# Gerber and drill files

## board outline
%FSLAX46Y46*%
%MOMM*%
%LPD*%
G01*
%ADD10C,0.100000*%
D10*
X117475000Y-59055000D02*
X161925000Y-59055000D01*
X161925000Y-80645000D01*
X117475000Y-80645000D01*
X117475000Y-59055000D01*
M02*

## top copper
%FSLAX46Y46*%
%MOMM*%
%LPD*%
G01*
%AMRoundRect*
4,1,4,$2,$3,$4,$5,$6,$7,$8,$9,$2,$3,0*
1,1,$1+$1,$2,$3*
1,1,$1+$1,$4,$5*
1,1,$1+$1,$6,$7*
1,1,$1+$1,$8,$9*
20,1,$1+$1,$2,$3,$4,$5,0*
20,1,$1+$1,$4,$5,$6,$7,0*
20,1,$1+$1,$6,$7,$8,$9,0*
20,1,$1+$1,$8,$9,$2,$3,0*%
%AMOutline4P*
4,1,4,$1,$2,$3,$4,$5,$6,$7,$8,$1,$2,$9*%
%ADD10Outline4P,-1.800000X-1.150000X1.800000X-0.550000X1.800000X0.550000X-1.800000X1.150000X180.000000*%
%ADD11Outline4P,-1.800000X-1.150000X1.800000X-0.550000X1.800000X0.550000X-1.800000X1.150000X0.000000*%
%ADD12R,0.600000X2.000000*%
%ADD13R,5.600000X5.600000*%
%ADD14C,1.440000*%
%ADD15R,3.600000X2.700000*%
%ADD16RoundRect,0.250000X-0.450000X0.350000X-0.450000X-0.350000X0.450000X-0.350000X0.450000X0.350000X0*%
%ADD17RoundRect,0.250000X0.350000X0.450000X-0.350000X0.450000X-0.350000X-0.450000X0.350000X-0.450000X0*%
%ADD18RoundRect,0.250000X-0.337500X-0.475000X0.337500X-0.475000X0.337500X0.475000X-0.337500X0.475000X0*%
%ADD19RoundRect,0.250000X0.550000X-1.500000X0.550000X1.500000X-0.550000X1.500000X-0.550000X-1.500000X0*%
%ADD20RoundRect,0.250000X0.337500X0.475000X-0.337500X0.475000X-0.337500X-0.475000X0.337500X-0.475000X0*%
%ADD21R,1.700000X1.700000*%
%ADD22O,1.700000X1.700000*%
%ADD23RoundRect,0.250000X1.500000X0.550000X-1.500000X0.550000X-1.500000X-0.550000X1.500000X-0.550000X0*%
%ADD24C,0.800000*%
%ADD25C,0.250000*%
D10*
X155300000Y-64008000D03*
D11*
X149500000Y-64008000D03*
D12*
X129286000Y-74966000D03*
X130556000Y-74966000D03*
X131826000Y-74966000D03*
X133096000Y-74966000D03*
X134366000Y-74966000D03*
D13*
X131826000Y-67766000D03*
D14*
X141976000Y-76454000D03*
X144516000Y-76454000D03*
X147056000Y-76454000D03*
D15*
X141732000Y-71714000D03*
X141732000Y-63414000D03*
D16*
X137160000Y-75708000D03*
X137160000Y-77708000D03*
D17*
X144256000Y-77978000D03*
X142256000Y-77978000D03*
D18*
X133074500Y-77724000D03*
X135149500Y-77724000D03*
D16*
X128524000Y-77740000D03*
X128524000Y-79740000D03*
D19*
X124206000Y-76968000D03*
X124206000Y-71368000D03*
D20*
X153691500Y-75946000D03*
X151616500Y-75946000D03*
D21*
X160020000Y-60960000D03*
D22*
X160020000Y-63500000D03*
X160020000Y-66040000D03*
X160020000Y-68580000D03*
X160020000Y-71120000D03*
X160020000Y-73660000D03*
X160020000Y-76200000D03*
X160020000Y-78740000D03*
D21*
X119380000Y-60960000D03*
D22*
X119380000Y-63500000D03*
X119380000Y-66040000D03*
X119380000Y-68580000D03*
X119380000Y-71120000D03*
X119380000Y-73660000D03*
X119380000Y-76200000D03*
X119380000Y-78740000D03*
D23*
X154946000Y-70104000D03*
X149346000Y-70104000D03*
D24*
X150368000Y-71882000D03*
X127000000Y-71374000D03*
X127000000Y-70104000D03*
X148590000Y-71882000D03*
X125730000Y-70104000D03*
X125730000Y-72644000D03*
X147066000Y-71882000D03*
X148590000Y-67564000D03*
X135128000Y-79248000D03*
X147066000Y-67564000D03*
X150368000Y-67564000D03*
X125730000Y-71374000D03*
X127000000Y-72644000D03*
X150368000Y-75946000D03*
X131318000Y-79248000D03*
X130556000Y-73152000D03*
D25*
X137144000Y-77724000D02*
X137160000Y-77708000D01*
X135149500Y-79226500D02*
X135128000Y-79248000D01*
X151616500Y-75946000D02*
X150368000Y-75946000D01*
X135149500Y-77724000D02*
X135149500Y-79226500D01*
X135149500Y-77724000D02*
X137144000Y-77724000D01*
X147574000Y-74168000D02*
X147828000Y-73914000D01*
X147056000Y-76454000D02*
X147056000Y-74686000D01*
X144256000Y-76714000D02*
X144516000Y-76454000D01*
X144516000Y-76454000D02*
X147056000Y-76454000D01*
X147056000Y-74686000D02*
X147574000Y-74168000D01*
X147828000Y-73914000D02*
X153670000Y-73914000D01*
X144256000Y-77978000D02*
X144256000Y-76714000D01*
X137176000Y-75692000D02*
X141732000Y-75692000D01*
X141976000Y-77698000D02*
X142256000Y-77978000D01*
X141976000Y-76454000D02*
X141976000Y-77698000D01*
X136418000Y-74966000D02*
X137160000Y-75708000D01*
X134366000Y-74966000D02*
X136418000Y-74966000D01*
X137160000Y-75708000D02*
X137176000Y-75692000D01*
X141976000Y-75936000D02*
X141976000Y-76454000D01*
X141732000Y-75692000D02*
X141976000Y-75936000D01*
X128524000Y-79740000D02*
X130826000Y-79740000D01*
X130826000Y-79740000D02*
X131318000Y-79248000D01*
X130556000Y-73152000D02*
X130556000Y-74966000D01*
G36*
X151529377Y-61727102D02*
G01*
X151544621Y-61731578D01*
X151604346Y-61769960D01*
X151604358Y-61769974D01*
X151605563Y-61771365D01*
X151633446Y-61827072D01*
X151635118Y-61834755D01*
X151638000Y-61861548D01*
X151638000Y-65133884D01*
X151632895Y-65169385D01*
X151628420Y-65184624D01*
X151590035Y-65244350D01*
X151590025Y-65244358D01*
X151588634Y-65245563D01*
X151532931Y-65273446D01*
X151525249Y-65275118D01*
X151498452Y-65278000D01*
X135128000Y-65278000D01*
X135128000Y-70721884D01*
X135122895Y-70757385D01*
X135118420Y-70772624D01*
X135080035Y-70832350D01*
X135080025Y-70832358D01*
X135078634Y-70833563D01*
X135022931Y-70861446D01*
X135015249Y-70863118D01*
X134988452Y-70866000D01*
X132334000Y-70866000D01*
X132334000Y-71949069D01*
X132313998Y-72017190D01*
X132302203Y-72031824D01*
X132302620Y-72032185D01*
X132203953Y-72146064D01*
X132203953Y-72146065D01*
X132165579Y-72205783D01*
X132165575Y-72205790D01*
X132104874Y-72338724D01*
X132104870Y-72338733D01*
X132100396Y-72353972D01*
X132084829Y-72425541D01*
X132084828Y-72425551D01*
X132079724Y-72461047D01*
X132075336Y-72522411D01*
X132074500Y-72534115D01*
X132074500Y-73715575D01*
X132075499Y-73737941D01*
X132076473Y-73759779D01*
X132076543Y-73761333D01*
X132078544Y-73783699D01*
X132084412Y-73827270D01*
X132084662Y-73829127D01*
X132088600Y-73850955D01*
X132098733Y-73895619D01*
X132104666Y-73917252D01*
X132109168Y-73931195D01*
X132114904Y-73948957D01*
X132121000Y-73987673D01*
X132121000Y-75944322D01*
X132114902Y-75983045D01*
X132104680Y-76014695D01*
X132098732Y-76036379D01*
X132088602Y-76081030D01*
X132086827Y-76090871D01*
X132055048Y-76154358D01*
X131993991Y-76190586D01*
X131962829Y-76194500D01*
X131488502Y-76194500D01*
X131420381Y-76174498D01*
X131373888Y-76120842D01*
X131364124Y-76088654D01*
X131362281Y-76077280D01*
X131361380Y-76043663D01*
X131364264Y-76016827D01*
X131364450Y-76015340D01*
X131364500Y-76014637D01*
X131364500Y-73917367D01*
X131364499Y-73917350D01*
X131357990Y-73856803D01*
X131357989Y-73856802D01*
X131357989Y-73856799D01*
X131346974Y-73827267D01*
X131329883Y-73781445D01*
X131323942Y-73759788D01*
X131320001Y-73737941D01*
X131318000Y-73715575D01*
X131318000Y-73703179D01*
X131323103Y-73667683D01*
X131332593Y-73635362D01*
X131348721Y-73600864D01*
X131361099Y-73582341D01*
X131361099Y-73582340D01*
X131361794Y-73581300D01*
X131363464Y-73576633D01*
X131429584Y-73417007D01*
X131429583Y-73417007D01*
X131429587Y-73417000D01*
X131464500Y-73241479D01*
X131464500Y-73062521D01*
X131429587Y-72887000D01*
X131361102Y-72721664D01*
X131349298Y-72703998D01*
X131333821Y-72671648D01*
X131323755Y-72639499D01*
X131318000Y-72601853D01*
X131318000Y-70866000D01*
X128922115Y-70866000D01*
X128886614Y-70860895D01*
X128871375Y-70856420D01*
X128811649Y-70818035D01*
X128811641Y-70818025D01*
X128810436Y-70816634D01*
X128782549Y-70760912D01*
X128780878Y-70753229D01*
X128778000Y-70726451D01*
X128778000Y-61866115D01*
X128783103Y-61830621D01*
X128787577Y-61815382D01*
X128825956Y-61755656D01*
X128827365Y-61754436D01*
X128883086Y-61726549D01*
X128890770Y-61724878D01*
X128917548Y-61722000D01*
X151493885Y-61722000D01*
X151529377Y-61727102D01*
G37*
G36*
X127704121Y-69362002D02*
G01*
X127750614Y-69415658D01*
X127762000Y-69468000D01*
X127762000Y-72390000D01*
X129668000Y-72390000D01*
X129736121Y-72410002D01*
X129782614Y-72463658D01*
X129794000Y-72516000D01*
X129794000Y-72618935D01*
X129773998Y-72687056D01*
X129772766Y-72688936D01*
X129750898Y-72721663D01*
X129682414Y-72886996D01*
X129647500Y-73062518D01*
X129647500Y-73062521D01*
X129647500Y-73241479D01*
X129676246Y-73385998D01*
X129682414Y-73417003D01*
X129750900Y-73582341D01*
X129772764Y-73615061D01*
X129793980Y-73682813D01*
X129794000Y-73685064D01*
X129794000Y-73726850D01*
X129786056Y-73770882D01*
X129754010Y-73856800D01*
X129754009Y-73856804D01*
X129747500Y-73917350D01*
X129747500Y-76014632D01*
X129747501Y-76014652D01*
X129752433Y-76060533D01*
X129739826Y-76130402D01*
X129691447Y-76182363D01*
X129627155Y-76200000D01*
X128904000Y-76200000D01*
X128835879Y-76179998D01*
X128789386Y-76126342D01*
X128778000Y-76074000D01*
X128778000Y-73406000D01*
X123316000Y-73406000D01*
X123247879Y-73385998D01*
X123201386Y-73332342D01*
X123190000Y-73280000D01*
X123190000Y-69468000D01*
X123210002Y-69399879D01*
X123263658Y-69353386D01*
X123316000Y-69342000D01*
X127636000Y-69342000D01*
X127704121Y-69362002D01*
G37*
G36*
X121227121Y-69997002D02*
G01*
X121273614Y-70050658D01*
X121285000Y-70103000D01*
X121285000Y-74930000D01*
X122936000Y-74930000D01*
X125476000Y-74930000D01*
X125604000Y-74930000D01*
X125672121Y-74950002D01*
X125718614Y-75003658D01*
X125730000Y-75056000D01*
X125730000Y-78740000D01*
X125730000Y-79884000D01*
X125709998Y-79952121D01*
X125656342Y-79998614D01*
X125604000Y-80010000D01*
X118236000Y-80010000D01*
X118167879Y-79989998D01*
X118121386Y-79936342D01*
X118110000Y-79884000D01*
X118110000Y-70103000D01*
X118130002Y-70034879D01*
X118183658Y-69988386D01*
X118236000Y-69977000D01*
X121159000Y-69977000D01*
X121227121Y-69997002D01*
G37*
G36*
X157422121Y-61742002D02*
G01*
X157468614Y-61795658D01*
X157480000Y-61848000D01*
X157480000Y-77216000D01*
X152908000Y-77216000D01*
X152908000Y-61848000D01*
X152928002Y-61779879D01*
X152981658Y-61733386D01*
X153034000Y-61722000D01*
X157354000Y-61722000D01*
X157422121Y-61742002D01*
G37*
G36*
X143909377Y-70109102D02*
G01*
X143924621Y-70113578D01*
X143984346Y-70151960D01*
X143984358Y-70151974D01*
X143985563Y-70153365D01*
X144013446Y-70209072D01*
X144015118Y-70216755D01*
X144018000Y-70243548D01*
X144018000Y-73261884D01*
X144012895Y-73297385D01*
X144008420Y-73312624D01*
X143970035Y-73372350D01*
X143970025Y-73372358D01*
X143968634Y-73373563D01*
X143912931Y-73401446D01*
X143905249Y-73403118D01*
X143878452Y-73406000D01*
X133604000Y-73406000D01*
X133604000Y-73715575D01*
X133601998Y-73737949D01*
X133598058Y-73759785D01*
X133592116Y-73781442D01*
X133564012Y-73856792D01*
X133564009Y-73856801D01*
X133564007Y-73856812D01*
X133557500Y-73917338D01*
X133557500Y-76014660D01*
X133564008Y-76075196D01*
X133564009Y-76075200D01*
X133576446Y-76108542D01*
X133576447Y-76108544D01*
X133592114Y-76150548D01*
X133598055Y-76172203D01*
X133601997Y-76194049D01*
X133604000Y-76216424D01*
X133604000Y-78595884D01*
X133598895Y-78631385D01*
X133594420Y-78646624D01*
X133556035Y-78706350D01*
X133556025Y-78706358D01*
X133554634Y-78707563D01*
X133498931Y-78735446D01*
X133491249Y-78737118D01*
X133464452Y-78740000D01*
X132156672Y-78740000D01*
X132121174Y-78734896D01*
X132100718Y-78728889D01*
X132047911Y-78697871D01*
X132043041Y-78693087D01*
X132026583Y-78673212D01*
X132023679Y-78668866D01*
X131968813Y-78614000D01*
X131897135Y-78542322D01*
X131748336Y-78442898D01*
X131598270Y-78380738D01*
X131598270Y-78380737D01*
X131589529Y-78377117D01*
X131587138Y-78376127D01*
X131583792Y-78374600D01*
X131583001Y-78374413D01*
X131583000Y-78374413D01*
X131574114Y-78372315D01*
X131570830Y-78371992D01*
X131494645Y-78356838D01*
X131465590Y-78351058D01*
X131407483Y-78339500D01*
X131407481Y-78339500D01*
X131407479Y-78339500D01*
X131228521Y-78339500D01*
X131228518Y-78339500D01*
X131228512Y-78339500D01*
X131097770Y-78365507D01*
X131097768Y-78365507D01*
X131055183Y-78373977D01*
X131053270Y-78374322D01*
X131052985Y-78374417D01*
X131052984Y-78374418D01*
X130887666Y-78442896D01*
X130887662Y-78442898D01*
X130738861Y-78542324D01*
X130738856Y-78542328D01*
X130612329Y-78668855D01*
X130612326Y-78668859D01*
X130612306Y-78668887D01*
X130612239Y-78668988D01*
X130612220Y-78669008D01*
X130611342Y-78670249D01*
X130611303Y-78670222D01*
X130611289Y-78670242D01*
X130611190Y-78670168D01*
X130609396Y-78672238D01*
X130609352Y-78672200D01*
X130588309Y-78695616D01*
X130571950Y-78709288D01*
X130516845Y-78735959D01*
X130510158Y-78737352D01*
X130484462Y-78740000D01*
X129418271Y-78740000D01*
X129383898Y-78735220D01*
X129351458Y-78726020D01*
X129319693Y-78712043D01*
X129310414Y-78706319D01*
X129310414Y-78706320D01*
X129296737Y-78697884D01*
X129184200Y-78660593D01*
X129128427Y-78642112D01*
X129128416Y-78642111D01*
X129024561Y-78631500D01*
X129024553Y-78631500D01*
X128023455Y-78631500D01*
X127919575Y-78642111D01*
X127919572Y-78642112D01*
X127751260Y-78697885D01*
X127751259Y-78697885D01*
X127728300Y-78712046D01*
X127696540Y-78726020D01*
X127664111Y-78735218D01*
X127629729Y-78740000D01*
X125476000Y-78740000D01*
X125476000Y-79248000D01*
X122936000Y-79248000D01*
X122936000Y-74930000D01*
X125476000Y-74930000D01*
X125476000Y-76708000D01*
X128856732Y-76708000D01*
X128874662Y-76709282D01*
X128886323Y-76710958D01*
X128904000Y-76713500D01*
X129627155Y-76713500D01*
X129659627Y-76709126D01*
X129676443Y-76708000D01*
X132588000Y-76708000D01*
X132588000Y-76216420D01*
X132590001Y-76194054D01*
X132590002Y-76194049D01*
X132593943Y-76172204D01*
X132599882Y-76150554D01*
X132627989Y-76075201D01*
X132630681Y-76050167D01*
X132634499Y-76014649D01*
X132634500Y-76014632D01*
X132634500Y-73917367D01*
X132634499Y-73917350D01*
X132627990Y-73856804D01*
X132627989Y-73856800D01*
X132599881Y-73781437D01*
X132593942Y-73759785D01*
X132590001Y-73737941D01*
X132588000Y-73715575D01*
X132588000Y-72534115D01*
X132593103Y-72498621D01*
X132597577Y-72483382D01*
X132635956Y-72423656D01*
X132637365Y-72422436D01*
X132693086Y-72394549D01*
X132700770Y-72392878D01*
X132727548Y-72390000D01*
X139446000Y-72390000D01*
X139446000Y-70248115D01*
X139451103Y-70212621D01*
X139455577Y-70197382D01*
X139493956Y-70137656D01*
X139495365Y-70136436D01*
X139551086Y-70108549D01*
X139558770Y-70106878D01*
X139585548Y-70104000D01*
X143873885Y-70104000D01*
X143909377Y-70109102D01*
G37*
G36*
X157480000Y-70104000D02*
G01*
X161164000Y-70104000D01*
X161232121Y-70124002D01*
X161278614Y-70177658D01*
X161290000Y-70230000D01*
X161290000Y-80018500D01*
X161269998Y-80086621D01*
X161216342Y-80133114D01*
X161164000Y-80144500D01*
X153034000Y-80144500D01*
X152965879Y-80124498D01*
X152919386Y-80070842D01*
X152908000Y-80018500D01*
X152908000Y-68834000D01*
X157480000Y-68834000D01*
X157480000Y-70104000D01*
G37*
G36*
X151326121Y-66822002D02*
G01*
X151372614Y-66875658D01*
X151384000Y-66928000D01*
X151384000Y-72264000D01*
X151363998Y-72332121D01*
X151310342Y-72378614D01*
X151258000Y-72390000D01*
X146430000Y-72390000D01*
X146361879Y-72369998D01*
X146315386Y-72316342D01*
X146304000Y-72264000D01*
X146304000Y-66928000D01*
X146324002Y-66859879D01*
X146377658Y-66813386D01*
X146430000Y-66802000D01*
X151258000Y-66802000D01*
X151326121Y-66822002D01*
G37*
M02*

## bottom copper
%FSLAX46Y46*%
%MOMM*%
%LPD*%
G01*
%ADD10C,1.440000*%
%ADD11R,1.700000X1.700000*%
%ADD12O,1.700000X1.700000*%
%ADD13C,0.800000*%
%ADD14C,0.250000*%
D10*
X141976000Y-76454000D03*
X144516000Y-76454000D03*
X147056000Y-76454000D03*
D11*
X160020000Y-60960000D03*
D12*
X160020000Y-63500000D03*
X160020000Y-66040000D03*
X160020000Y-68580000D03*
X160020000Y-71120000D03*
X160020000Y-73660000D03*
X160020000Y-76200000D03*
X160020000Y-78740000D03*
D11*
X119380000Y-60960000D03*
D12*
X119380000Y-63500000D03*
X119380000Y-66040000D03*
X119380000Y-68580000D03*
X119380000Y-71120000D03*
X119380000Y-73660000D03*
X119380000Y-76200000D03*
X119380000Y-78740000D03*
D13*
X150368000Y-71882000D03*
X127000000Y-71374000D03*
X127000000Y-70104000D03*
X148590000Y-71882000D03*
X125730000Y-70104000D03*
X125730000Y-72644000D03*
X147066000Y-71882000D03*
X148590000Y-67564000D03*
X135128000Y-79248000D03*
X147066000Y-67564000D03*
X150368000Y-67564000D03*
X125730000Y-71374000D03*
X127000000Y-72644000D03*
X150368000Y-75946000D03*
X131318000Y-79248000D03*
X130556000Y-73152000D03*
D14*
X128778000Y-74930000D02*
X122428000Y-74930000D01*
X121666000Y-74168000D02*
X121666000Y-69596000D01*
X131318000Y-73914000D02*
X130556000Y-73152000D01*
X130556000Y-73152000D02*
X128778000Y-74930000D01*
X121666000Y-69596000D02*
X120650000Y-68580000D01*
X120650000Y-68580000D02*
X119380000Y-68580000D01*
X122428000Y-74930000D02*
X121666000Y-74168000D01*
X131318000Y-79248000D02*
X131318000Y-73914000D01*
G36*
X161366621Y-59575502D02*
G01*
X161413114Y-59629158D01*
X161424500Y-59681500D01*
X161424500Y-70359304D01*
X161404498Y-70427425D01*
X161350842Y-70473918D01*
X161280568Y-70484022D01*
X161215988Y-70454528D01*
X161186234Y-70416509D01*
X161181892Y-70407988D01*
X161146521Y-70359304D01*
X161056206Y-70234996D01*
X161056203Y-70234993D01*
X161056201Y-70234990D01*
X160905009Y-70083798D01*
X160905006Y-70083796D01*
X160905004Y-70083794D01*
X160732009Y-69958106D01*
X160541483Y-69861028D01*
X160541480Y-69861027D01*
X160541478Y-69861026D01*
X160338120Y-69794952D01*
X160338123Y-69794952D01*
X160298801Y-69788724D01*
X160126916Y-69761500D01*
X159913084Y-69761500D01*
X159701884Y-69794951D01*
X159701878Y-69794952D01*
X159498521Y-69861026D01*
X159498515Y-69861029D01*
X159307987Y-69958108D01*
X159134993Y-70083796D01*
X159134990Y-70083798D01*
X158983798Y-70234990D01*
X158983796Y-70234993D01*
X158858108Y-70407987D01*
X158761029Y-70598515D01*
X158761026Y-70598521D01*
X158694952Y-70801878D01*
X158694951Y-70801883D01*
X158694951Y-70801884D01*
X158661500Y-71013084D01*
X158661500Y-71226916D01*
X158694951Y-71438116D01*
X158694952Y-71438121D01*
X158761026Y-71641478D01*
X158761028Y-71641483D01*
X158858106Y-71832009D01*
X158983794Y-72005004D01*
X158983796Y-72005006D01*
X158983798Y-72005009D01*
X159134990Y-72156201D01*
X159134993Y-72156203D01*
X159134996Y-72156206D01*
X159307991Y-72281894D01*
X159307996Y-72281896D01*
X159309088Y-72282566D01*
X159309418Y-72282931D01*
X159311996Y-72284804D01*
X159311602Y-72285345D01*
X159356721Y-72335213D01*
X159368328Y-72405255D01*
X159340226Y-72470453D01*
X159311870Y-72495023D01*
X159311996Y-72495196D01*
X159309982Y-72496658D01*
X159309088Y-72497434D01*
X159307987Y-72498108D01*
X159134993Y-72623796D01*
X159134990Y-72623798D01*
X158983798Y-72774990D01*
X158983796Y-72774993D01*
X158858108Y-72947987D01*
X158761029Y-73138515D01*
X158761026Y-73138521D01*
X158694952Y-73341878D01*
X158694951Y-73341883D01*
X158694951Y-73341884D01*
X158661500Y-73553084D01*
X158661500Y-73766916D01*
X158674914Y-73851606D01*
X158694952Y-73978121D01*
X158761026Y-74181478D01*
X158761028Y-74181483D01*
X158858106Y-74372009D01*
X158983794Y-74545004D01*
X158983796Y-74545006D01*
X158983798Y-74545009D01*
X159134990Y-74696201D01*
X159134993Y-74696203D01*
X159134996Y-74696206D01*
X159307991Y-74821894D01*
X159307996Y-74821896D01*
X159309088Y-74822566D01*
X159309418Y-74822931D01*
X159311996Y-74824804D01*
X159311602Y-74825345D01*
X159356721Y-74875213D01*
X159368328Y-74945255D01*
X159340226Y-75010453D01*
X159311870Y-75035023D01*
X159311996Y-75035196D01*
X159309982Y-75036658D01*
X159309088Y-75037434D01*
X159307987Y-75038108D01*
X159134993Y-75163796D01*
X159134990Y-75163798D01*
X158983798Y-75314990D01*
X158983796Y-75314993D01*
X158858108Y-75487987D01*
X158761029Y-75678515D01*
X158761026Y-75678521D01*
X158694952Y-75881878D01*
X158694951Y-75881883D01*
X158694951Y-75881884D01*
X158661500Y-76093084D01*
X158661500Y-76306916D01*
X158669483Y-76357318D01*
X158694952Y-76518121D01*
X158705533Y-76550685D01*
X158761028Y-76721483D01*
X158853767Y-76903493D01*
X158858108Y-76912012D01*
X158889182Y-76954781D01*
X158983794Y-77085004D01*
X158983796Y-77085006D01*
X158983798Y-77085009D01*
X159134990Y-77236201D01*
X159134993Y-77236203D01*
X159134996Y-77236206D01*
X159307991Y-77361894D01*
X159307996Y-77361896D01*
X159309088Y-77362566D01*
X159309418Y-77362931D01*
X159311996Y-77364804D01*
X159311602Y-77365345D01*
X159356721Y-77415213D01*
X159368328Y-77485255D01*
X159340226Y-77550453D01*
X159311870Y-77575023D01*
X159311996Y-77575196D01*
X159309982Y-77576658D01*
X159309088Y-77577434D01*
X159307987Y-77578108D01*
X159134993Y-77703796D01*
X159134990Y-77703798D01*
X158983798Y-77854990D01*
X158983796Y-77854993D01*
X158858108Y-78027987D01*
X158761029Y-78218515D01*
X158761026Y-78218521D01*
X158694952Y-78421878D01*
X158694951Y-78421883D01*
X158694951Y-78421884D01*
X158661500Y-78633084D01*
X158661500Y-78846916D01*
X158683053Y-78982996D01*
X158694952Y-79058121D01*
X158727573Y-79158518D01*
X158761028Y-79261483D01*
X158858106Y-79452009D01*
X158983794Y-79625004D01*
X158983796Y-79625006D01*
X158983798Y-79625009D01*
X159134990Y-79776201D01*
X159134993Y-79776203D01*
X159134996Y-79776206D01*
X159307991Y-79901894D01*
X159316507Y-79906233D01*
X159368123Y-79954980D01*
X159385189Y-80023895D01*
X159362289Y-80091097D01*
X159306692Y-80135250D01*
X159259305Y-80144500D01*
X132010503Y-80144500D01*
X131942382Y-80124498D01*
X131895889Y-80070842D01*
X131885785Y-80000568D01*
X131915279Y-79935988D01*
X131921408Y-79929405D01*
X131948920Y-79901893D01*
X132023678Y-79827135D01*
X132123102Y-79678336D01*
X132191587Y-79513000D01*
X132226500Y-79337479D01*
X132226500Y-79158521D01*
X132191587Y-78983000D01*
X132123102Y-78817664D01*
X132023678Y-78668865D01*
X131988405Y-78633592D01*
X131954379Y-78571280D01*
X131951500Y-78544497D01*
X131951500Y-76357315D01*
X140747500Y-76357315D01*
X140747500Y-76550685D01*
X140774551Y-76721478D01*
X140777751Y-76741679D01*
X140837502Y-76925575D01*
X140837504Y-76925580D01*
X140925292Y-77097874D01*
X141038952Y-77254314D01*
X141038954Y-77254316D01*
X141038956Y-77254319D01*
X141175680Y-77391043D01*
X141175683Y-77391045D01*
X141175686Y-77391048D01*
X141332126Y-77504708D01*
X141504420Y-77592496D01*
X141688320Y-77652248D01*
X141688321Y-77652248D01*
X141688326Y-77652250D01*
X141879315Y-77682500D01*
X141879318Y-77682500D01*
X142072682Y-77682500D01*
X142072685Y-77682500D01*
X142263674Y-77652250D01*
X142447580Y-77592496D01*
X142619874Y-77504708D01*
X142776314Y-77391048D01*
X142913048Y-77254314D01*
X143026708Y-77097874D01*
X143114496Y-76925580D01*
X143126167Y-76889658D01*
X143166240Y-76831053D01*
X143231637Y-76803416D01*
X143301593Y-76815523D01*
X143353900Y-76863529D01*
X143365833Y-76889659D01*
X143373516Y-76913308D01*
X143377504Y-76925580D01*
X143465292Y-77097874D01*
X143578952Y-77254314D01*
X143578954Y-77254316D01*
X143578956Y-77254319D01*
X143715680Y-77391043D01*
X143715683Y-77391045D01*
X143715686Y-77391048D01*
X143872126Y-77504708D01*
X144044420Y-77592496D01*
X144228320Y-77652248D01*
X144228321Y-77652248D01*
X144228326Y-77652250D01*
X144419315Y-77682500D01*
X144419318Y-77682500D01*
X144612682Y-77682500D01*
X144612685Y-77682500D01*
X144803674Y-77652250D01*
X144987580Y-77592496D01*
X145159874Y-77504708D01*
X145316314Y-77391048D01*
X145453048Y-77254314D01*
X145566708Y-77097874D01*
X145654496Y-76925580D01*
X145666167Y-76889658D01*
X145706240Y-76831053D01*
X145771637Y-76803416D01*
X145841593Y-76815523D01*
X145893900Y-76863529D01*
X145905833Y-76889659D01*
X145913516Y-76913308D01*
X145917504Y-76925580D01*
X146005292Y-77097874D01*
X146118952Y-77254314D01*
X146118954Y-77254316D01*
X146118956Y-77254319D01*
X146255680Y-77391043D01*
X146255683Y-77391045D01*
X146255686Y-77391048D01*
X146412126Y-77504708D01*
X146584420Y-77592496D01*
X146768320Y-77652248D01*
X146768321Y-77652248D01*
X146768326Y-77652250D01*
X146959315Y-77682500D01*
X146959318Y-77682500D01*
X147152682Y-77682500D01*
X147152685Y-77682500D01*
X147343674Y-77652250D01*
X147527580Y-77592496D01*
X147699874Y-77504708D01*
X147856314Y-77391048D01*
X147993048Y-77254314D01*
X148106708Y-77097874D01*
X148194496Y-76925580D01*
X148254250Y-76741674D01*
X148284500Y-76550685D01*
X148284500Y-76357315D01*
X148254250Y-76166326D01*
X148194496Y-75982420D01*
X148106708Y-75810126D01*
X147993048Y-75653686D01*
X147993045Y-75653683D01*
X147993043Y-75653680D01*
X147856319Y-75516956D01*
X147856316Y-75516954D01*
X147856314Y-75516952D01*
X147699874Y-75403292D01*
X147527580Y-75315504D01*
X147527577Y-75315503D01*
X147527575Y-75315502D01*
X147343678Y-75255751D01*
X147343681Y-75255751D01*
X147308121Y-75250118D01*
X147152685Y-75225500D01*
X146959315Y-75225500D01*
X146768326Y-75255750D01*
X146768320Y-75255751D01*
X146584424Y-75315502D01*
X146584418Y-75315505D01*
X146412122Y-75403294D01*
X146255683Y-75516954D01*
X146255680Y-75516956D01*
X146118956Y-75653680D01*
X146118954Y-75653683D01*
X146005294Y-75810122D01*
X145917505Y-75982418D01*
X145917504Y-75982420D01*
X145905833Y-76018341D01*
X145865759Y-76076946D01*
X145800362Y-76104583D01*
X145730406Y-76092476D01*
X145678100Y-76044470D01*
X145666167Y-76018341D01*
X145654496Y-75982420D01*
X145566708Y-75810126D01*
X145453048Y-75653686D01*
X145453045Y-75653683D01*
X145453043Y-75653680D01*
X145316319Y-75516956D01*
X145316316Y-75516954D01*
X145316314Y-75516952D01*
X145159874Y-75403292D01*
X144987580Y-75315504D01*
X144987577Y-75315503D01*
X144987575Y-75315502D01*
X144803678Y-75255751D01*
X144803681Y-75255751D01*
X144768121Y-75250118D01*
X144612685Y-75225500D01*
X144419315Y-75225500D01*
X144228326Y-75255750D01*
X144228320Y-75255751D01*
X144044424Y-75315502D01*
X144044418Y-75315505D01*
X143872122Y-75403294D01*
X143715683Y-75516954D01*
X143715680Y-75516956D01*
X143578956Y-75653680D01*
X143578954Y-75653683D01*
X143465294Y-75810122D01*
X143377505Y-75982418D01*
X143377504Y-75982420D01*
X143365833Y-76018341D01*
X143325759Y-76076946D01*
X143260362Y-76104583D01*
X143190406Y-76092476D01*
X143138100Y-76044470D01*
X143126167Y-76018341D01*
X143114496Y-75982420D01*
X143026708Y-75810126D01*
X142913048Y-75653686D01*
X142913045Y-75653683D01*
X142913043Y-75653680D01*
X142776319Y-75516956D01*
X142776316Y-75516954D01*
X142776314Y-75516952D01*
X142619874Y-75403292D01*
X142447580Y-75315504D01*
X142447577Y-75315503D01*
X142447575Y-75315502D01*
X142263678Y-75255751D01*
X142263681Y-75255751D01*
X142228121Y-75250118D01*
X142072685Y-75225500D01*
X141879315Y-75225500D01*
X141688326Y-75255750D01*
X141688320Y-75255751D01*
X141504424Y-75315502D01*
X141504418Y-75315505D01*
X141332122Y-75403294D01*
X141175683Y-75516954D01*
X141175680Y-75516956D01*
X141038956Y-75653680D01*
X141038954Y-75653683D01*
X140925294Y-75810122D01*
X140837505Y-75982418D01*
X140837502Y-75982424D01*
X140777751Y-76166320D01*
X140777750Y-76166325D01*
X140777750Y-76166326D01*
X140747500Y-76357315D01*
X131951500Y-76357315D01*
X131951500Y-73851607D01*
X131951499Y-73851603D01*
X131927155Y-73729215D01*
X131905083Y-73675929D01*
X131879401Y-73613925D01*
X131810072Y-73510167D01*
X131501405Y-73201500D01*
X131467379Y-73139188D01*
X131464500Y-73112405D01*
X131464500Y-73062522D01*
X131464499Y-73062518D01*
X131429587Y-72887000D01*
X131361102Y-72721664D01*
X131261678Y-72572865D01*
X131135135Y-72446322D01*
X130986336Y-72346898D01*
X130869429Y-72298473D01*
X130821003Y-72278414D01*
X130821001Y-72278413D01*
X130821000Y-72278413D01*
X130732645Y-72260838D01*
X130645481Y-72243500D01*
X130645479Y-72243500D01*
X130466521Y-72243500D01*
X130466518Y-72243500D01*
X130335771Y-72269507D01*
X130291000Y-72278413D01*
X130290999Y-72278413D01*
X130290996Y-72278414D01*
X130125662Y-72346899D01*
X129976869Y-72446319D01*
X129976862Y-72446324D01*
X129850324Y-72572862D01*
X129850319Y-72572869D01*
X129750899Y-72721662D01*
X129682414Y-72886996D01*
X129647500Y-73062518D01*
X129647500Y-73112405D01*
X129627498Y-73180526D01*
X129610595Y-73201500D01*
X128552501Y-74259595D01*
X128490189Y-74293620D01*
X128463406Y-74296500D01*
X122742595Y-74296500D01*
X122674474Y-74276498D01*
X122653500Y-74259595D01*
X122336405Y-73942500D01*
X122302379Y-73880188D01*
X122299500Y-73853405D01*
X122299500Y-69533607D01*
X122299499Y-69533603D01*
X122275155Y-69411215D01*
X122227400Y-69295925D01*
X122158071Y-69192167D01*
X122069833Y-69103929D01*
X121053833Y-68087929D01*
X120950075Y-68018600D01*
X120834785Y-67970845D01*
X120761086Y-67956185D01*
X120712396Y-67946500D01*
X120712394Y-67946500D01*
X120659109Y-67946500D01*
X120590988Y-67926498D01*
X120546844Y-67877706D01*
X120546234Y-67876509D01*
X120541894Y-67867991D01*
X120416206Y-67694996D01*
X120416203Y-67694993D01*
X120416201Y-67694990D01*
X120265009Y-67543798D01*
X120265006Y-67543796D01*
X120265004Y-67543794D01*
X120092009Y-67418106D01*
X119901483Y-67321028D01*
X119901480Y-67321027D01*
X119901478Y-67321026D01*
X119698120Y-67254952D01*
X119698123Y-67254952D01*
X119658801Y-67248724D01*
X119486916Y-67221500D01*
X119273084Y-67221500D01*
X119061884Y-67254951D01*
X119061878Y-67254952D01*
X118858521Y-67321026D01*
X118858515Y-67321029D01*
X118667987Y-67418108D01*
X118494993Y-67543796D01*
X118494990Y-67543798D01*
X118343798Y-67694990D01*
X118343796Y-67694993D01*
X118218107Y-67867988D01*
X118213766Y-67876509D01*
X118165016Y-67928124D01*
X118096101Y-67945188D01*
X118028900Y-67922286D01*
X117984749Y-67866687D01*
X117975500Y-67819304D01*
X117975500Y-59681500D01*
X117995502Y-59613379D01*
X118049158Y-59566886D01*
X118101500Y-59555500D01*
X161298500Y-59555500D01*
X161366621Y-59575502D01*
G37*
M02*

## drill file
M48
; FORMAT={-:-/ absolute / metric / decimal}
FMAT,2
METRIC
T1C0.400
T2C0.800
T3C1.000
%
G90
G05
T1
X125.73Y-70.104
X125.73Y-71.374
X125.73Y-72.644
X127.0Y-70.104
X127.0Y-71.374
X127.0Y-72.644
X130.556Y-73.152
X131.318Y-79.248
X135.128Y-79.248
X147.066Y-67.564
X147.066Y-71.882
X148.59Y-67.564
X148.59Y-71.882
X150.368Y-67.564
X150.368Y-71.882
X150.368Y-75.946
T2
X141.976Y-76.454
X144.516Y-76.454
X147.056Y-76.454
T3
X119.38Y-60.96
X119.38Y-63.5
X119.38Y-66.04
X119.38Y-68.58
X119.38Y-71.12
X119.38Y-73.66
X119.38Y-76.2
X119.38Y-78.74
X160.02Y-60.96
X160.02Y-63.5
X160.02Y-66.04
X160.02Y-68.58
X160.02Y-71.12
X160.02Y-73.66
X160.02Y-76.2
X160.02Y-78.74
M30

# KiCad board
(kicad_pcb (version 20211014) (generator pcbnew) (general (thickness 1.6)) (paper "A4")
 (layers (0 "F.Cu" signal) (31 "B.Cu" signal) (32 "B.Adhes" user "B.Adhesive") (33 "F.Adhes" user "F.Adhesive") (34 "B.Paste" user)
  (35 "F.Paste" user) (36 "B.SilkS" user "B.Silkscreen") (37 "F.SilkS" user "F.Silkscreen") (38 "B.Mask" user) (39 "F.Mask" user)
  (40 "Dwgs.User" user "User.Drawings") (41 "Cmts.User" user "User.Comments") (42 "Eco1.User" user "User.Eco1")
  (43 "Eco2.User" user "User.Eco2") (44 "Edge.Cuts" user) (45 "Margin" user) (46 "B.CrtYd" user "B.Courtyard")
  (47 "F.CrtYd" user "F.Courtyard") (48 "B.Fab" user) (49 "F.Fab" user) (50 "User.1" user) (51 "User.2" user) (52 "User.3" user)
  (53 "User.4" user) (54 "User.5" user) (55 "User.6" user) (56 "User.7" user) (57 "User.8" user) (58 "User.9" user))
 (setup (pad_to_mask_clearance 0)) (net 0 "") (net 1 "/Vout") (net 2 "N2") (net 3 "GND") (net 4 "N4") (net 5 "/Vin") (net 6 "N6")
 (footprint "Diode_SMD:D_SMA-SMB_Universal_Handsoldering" (layer "F.Cu") (at 152.4 64.008 180)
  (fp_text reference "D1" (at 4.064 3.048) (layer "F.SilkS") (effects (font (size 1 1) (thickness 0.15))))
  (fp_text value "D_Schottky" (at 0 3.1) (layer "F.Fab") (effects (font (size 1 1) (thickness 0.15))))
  (pad "1" smd trapezoid locked (at -2.9 0 180) (size 3.6 1.7) (rect_delta 0.6 0) (layers "F.Cu" "F.Paste" "F.Mask") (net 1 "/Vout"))
  (pad "2" smd trapezoid locked (at 2.9 0) (size 3.6 1.7) (rect_delta 0.6 0) (layers "F.Cu" "F.Paste" "F.Mask") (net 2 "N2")))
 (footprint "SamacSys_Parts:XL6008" (layer "F.Cu") (at 131.826 74.966)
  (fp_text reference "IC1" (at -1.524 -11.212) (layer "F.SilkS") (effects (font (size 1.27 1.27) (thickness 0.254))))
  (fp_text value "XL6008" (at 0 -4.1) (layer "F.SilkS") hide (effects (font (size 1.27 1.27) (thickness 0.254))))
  (pad "1" smd rect locked (at -2.54 0) (size 0.6 2) (layers "F.Cu" "F.Paste" "F.Mask") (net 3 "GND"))
  (pad "2" smd rect locked (at -1.27 0) (size 0.6 2) (layers "F.Cu" "F.Paste" "F.Mask") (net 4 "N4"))
  (pad "3" smd rect locked (at 0 0) (size 0.6 2) (layers "F.Cu" "F.Paste" "F.Mask") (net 2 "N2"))
  (pad "4" smd rect locked (at 1.27 0) (size 0.6 2) (layers "F.Cu" "F.Paste" "F.Mask") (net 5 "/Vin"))
  (pad "5" smd rect locked (at 2.54 0) (size 0.6 2) (layers "F.Cu" "F.Paste" "F.Mask") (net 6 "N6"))
  (pad "6" smd rect locked (at 0 -7.2 90) (size 5.6 5.6) (layers "F.Cu" "F.Paste" "F.Mask") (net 2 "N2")))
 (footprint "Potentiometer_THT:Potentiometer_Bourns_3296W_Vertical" (layer "F.Cu") (at 141.976 76.454 180)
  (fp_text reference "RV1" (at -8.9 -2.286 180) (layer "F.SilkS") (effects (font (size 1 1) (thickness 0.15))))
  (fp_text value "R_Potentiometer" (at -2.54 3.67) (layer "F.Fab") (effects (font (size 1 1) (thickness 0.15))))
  (pad "1" thru_hole circle locked (at 0 0 180) (size 1.44 1.44) (drill 0.8) (layers *.Cu *.Mask) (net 6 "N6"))
  (pad "2" thru_hole circle locked (at -2.54 0 180) (size 1.44 1.44) (drill 0.8) (layers *.Cu *.Mask) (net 1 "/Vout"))
  (pad "3" thru_hole circle locked (at -5.08 0 180) (size 1.44 1.44) (drill 0.8) (layers *.Cu *.Mask) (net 1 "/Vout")))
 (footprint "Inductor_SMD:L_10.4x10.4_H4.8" (layer "F.Cu") (at 141.732 67.564 90)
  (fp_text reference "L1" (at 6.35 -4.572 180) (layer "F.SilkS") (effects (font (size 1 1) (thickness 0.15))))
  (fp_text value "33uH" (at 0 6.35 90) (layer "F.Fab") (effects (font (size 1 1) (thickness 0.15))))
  (pad "1" smd rect locked (at -4.15 0 90) (size 2.7 3.6) (layers "F.Cu" "F.Paste" "F.Mask") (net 5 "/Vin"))
  (pad "2" smd rect locked (at 4.15 0 90) (size 2.7 3.6) (layers "F.Cu" "F.Paste" "F.Mask") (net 2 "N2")))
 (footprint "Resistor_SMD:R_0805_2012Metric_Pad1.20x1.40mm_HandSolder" (layer "F.Cu") (at 137.16 76.708 -90)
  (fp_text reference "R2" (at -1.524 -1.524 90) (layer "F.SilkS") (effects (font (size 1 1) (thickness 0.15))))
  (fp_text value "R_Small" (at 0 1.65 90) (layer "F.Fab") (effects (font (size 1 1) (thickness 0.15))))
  (pad "1" smd roundrect locked (at -1 0 270) (size 1.2 1.4) (layers "F.Cu" "F.Paste" "F.Mask") (roundrect_rratio 0.208333) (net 6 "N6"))
  (pad "2" smd roundrect locked (at 1 0 270) (size 1.2 1.4) (layers "F.Cu" "F.Paste" "F.Mask") (roundrect_rratio 0.208333) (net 3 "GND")))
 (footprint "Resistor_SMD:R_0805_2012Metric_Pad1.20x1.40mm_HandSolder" (layer "F.Cu") (at 143.256 77.978 180)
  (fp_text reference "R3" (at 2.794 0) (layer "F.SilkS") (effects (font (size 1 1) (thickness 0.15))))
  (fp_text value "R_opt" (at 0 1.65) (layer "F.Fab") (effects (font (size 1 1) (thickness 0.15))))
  (pad "1" smd roundrect locked (at -1 0 180) (size 1.2 1.4) (layers "F.Cu" "F.Paste" "F.Mask") (roundrect_rratio 0.208333) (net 1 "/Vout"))
  (pad "2" smd roundrect locked (at 1 0 180) (size 1.2 1.4) (layers "F.Cu" "F.Paste" "F.Mask") (roundrect_rratio 0.208333) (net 6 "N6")))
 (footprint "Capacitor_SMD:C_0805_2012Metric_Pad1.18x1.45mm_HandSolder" (layer "F.Cu") (at 134.112 77.724)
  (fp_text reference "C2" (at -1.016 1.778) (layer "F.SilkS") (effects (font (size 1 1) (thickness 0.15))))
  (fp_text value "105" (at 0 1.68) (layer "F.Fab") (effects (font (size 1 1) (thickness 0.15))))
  (pad "1" smd roundrect locked (at -1.0375 0) (size 1.175 1.45) (layers "F.Cu" "F.Paste" "F.Mask") (roundrect_rratio 0.212766)
   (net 5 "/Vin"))
  (pad "2" smd roundrect locked (at 1.0375 0) (size 1.175 1.45) (layers "F.Cu" "F.Paste" "F.Mask") (roundrect_rratio 0.212766) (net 3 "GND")))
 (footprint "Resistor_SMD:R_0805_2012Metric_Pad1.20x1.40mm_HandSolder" (layer "F.Cu") (at 128.524 78.74 -90)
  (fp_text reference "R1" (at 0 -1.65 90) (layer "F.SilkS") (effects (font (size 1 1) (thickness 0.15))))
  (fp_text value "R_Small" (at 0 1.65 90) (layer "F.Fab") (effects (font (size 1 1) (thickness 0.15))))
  (pad "1" smd roundrect locked (at -1 0 270) (size 1.2 1.4) (layers "F.Cu" "F.Paste" "F.Mask") (roundrect_rratio 0.208333) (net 5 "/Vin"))
  (pad "2" smd roundrect locked (at 1 0 270) (size 1.2 1.4) (layers "F.Cu" "F.Paste" "F.Mask") (roundrect_rratio 0.208333) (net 4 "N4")))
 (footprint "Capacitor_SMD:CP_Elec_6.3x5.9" (layer "F.Cu") (at 124.206 74.168 90)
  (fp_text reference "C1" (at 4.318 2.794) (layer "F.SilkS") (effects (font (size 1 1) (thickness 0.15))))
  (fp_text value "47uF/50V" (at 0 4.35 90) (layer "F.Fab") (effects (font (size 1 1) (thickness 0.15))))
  (pad "1" smd roundrect locked (at -2.8 0 90) (size 3.5 1.6) (layers "F.Cu" "F.Paste" "F.Mask") (roundrect_rratio 0.15625) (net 5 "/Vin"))
  (pad "2" smd roundrect locked (at 2.8 0 90) (size 3.5 1.6) (layers "F.Cu" "F.Paste" "F.Mask") (roundrect_rratio 0.15625) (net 3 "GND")))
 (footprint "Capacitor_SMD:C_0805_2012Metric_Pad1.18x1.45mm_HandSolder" (layer "F.Cu") (at 152.654 75.946 180)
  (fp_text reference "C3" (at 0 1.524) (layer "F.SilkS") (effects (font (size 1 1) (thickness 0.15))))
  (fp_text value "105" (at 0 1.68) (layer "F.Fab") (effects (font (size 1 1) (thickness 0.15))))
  (pad "1" smd roundrect locked (at -1.0375 0 180) (size 1.175 1.45) (layers "F.Cu" "F.Paste" "F.Mask") (roundrect_rratio 0.212766)
   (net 1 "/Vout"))
  (pad "2" smd roundrect locked (at 1.0375 0 180) (size 1.175 1.45) (layers "F.Cu" "F.Paste" "F.Mask") (roundrect_rratio 0.212766)
   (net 3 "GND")))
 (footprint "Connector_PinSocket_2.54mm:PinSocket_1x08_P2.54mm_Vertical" (layer "F.Cu") (at 160.02 60.96)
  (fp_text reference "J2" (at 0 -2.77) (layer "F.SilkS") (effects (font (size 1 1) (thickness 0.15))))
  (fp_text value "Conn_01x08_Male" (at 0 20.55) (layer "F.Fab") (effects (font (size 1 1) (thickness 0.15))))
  (pad "1" thru_hole rect locked (at 0 0) (size 1.7 1.7) (drill 1) (layers *.Cu *.Mask) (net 3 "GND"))
  (pad "2" thru_hole oval locked (at 0 2.54) (size 1.7 1.7) (drill 1) (layers *.Cu *.Mask) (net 3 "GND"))
  (pad "3" thru_hole oval locked (at 0 5.08) (size 1.7 1.7) (drill 1) (layers *.Cu *.Mask) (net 3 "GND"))
  (pad "4" thru_hole oval locked (at 0 7.62) (size 1.7 1.7) (drill 1) (layers *.Cu *.Mask) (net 3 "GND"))
  (pad "5" thru_hole oval locked (at 0 10.16) (size 1.7 1.7) (drill 1) (layers *.Cu *.Mask) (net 1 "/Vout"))
  (pad "6" thru_hole oval locked (at 0 12.7) (size 1.7 1.7) (drill 1) (layers *.Cu *.Mask) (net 1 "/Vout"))
  (pad "7" thru_hole oval locked (at 0 15.24) (size 1.7 1.7) (drill 1) (layers *.Cu *.Mask) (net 1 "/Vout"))
  (pad "8" thru_hole oval locked (at 0 17.78) (size 1.7 1.7) (drill 1) (layers *.Cu *.Mask) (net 1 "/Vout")))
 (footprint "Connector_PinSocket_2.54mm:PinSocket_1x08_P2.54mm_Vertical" (layer "F.Cu") (at 119.38 60.96)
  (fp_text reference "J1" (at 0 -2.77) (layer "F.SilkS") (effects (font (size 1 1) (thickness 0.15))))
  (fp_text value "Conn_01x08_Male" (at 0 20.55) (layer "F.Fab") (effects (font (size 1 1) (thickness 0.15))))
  (pad "1" thru_hole rect locked (at 0 0) (size 1.7 1.7) (drill 1) (layers *.Cu *.Mask) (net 3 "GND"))
  (pad "2" thru_hole oval locked (at 0 2.54) (size 1.7 1.7) (drill 1) (layers *.Cu *.Mask) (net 3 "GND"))
  (pad "3" thru_hole oval locked (at 0 5.08) (size 1.7 1.7) (drill 1) (layers *.Cu *.Mask) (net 3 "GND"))
  (pad "4" thru_hole oval locked (at 0 7.62) (size 1.7 1.7) (drill 1) (layers *.Cu *.Mask) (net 4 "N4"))
  (pad "5" thru_hole oval locked (at 0 10.16) (size 1.7 1.7) (drill 1) (layers *.Cu *.Mask) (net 5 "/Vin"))
  (pad "6" thru_hole oval locked (at 0 12.7) (size 1.7 1.7) (drill 1) (layers *.Cu *.Mask) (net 5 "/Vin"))
  (pad "7" thru_hole oval locked (at 0 15.24) (size 1.7 1.7) (drill 1) (layers *.Cu *.Mask) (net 5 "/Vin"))
  (pad "8" thru_hole oval locked (at 0 17.78) (size 1.7 1.7) (drill 1) (layers *.Cu *.Mask) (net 5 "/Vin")))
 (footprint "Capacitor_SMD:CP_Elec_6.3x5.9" (layer "F.Cu") (at 152.146 70.104 180)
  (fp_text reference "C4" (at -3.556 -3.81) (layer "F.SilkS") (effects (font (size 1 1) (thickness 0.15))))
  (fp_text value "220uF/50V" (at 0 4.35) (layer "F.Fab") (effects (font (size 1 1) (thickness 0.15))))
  (pad "1" smd roundrect locked (at -2.8 0 180) (size 3.5 1.6) (layers "F.Cu" "F.Paste" "F.Mask") (roundrect_rratio 0.15625) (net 1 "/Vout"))
  (pad "2" smd roundrect locked (at 2.8 0 180) (size 3.5 1.6) (layers "F.Cu" "F.Paste" "F.Mask") (roundrect_rratio 0.15625) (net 3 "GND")))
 (gr_rect (start 117.475 59.055) (end 161.925 80.645) (layer "Edge.Cuts") (width 0.1) (fill none))
 (segment (start 137.144 77.724) (end 137.16 77.708) (width 0.25) (layer "F.Cu") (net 3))
 (segment (start 135.1495 79.2265) (end 135.128 79.248) (width 0.25) (layer "F.Cu") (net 3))
 (segment (start 151.6165 75.946) (end 150.368 75.946) (width 0.25) (layer "F.Cu") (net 3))
 (segment (start 135.1495 77.724) (end 135.1495 79.2265) (width 0.25) (layer "F.Cu") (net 3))
 (segment (start 135.1495 77.724) (end 137.144 77.724) (width 0.25) (layer "F.Cu") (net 3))
 (via (at 150.368 71.882) (size 0.8) (drill 0.4) (layers "F.Cu" "B.Cu") (free) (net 3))
 (via (at 127 71.374) (size 0.8) (drill 0.4) (layers "F.Cu" "B.Cu") (free) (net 3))
 (via (at 127 70.104) (size 0.8) (drill 0.4) (layers "F.Cu" "B.Cu") (free) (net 3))
 (via (at 148.59 71.882) (size 0.8) (drill 0.4) (layers "F.Cu" "B.Cu") (free) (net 3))
 (via (at 125.73 70.104) (size 0.8) (drill 0.4) (layers "F.Cu" "B.Cu") (free) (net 3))
 (via (at 125.73 72.644) (size 0.8) (drill 0.4) (layers "F.Cu" "B.Cu") (free) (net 3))
 (via (at 147.066 71.882) (size 0.8) (drill 0.4) (layers "F.Cu" "B.Cu") (free) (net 3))
 (via (at 148.59 67.564) (size 0.8) (drill 0.4) (layers "F.Cu" "B.Cu") (free) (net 3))
 (via (at 135.128 79.248) (size 0.8) (drill 0.4) (layers "F.Cu" "B.Cu") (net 3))
 (via (at 147.066 67.564) (size 0.8) (drill 0.4) (layers "F.Cu" "B.Cu") (free) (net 3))
 (via (at 150.368 67.564) (size 0.8) (drill 0.4) (layers "F.Cu" "B.Cu") (free) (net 3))
 (via (at 125.73 71.374) (size 0.8) (drill 0.4) (layers "F.Cu" "B.Cu") (free) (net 3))
 (via (at 127 72.644) (size 0.8) (drill 0.4) (layers "F.Cu" "B.Cu") (free) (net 3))
 (via (at 150.368 75.946) (size 0.8) (drill 0.4) (layers "F.Cu" "B.Cu") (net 3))
 (segment (start 147.574 74.168) (end 147.828 73.914) (width 0.25) (layer "F.Cu") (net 1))
 (segment (start 147.056 76.454) (end 147.056 74.686) (width 0.25) (layer "F.Cu") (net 1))
 (segment (start 144.256 76.714) (end 144.516 76.454) (width 0.25) (layer "F.Cu") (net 1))
 (segment (start 144.516 76.454) (end 147.056 76.454) (width 0.25) (layer "F.Cu") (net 1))
 (segment (start 147.056 74.686) (end 147.574 74.168) (width 0.25) (layer "F.Cu") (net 1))
 (segment (start 147.828 73.914) (end 153.67 73.914) (width 0.25) (layer "F.Cu") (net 1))
 (segment (start 144.256 77.978) (end 144.256 76.714) (width 0.25) (layer "F.Cu") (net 1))
 (segment (start 137.176 75.692) (end 141.732 75.692) (width 0.25) (layer "F.Cu") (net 6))
 (segment (start 141.976 77.698) (end 142.256 77.978) (width 0.25) (layer "F.Cu") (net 6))
 (segment (start 141.976 76.454) (end 141.976 77.698) (width 0.25) (layer "F.Cu") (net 6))
 (segment (start 136.418 74.966) (end 137.16 75.708) (width 0.25) (layer "F.Cu") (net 6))
 (segment (start 134.366 74.966) (end 136.418 74.966) (width 0.25) (layer "F.Cu") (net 6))
 (segment (start 137.16 75.708) (end 137.176 75.692) (width 0.25) (layer "F.Cu") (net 6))
 (segment (start 141.976 75.936) (end 141.976 76.454) (width 0.25) (layer "F.Cu") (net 6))
 (segment (start 141.732 75.692) (end 141.976 75.936) (width 0.25) (layer "F.Cu") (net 6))
 (segment (start 128.524 79.74) (end 130.826 79.74) (width 0.25) (layer "F.Cu") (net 4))
 (segment (start 130.826 79.74) (end 131.318 79.248) (width 0.25) (layer "F.Cu") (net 4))
 (segment (start 130.556 73.152) (end 130.556 74.966) (width 0.25) (layer "F.Cu") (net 4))
 (via (at 131.318 79.248) (size 0.8) (drill 0.4) (layers "F.Cu" "B.Cu") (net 4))
 (via (at 130.556 73.152) (size 0.8) (drill 0.4) (layers "F.Cu" "B.Cu") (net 4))
 (segment (start 128.778 74.93) (end 122.428 74.93) (width 0.25) (layer "B.Cu") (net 4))
 (segment (start 121.666 74.168) (end 121.666 69.596) (width 0.25) (layer "B.Cu") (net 4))
 (segment (start 131.318 73.914) (end 130.556 73.152) (width 0.25) (layer "B.Cu") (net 4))
 (segment (start 130.556 73.152) (end 128.778 74.93) (width 0.25) (layer "B.Cu") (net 4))
 (segment (start 121.666 69.596) (end 120.65 68.58) (width 0.25) (layer "B.Cu") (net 4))
 (segment (start 120.65 68.58) (end 119.38 68.58) (width 0.25) (layer "B.Cu") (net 4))
 (segment (start 122.428 74.93) (end 121.666 74.168) (width 0.25) (layer "B.Cu") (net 4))
 (segment (start 131.318 79.248) (end 131.318 73.914) (width 0.25) (layer "B.Cu") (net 4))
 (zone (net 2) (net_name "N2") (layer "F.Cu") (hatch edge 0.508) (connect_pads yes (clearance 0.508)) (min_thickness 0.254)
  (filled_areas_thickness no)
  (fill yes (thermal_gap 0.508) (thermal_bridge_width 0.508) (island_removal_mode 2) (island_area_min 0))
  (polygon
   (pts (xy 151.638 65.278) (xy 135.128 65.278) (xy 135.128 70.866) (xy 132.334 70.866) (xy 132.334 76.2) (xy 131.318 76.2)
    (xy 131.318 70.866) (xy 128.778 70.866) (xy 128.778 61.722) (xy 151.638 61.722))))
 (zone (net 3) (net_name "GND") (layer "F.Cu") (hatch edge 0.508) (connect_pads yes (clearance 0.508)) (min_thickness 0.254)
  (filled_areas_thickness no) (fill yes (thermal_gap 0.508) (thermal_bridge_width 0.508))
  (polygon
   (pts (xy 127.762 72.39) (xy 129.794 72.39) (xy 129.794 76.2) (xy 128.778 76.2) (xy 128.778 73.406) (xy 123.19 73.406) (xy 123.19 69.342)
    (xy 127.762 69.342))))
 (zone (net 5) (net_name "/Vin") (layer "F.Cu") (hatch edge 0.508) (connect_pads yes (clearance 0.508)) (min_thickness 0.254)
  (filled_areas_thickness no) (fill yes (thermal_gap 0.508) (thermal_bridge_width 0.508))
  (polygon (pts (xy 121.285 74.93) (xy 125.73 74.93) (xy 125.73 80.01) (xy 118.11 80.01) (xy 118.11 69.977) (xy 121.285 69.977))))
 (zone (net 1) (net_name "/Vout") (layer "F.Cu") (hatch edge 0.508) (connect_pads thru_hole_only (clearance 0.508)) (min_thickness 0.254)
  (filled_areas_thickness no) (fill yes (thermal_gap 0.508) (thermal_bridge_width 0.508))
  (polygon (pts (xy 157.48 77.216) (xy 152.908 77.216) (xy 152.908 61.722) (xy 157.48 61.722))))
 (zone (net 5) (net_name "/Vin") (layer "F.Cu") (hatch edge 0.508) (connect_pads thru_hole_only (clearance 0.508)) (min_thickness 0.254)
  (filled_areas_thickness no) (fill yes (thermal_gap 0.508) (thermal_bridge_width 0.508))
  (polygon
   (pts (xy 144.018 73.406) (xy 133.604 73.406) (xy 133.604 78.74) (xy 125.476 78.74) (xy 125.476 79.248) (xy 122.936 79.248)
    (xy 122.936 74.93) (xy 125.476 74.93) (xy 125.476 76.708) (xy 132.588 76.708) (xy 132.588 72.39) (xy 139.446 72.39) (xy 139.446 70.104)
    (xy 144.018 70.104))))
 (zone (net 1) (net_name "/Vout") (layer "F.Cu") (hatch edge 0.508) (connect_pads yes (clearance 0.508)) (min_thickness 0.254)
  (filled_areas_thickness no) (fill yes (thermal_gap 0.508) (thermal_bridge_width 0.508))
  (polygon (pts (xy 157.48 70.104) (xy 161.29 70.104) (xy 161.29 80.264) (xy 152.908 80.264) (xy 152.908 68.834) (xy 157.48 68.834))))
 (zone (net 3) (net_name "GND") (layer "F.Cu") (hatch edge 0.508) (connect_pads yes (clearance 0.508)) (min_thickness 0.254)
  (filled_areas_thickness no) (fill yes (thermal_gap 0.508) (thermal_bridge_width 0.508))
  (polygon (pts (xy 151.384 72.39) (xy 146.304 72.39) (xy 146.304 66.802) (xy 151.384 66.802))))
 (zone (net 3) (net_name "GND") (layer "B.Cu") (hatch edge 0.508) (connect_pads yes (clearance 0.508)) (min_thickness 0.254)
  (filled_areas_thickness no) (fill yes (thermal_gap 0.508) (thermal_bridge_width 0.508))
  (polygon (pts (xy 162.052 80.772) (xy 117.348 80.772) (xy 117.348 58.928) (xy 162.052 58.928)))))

